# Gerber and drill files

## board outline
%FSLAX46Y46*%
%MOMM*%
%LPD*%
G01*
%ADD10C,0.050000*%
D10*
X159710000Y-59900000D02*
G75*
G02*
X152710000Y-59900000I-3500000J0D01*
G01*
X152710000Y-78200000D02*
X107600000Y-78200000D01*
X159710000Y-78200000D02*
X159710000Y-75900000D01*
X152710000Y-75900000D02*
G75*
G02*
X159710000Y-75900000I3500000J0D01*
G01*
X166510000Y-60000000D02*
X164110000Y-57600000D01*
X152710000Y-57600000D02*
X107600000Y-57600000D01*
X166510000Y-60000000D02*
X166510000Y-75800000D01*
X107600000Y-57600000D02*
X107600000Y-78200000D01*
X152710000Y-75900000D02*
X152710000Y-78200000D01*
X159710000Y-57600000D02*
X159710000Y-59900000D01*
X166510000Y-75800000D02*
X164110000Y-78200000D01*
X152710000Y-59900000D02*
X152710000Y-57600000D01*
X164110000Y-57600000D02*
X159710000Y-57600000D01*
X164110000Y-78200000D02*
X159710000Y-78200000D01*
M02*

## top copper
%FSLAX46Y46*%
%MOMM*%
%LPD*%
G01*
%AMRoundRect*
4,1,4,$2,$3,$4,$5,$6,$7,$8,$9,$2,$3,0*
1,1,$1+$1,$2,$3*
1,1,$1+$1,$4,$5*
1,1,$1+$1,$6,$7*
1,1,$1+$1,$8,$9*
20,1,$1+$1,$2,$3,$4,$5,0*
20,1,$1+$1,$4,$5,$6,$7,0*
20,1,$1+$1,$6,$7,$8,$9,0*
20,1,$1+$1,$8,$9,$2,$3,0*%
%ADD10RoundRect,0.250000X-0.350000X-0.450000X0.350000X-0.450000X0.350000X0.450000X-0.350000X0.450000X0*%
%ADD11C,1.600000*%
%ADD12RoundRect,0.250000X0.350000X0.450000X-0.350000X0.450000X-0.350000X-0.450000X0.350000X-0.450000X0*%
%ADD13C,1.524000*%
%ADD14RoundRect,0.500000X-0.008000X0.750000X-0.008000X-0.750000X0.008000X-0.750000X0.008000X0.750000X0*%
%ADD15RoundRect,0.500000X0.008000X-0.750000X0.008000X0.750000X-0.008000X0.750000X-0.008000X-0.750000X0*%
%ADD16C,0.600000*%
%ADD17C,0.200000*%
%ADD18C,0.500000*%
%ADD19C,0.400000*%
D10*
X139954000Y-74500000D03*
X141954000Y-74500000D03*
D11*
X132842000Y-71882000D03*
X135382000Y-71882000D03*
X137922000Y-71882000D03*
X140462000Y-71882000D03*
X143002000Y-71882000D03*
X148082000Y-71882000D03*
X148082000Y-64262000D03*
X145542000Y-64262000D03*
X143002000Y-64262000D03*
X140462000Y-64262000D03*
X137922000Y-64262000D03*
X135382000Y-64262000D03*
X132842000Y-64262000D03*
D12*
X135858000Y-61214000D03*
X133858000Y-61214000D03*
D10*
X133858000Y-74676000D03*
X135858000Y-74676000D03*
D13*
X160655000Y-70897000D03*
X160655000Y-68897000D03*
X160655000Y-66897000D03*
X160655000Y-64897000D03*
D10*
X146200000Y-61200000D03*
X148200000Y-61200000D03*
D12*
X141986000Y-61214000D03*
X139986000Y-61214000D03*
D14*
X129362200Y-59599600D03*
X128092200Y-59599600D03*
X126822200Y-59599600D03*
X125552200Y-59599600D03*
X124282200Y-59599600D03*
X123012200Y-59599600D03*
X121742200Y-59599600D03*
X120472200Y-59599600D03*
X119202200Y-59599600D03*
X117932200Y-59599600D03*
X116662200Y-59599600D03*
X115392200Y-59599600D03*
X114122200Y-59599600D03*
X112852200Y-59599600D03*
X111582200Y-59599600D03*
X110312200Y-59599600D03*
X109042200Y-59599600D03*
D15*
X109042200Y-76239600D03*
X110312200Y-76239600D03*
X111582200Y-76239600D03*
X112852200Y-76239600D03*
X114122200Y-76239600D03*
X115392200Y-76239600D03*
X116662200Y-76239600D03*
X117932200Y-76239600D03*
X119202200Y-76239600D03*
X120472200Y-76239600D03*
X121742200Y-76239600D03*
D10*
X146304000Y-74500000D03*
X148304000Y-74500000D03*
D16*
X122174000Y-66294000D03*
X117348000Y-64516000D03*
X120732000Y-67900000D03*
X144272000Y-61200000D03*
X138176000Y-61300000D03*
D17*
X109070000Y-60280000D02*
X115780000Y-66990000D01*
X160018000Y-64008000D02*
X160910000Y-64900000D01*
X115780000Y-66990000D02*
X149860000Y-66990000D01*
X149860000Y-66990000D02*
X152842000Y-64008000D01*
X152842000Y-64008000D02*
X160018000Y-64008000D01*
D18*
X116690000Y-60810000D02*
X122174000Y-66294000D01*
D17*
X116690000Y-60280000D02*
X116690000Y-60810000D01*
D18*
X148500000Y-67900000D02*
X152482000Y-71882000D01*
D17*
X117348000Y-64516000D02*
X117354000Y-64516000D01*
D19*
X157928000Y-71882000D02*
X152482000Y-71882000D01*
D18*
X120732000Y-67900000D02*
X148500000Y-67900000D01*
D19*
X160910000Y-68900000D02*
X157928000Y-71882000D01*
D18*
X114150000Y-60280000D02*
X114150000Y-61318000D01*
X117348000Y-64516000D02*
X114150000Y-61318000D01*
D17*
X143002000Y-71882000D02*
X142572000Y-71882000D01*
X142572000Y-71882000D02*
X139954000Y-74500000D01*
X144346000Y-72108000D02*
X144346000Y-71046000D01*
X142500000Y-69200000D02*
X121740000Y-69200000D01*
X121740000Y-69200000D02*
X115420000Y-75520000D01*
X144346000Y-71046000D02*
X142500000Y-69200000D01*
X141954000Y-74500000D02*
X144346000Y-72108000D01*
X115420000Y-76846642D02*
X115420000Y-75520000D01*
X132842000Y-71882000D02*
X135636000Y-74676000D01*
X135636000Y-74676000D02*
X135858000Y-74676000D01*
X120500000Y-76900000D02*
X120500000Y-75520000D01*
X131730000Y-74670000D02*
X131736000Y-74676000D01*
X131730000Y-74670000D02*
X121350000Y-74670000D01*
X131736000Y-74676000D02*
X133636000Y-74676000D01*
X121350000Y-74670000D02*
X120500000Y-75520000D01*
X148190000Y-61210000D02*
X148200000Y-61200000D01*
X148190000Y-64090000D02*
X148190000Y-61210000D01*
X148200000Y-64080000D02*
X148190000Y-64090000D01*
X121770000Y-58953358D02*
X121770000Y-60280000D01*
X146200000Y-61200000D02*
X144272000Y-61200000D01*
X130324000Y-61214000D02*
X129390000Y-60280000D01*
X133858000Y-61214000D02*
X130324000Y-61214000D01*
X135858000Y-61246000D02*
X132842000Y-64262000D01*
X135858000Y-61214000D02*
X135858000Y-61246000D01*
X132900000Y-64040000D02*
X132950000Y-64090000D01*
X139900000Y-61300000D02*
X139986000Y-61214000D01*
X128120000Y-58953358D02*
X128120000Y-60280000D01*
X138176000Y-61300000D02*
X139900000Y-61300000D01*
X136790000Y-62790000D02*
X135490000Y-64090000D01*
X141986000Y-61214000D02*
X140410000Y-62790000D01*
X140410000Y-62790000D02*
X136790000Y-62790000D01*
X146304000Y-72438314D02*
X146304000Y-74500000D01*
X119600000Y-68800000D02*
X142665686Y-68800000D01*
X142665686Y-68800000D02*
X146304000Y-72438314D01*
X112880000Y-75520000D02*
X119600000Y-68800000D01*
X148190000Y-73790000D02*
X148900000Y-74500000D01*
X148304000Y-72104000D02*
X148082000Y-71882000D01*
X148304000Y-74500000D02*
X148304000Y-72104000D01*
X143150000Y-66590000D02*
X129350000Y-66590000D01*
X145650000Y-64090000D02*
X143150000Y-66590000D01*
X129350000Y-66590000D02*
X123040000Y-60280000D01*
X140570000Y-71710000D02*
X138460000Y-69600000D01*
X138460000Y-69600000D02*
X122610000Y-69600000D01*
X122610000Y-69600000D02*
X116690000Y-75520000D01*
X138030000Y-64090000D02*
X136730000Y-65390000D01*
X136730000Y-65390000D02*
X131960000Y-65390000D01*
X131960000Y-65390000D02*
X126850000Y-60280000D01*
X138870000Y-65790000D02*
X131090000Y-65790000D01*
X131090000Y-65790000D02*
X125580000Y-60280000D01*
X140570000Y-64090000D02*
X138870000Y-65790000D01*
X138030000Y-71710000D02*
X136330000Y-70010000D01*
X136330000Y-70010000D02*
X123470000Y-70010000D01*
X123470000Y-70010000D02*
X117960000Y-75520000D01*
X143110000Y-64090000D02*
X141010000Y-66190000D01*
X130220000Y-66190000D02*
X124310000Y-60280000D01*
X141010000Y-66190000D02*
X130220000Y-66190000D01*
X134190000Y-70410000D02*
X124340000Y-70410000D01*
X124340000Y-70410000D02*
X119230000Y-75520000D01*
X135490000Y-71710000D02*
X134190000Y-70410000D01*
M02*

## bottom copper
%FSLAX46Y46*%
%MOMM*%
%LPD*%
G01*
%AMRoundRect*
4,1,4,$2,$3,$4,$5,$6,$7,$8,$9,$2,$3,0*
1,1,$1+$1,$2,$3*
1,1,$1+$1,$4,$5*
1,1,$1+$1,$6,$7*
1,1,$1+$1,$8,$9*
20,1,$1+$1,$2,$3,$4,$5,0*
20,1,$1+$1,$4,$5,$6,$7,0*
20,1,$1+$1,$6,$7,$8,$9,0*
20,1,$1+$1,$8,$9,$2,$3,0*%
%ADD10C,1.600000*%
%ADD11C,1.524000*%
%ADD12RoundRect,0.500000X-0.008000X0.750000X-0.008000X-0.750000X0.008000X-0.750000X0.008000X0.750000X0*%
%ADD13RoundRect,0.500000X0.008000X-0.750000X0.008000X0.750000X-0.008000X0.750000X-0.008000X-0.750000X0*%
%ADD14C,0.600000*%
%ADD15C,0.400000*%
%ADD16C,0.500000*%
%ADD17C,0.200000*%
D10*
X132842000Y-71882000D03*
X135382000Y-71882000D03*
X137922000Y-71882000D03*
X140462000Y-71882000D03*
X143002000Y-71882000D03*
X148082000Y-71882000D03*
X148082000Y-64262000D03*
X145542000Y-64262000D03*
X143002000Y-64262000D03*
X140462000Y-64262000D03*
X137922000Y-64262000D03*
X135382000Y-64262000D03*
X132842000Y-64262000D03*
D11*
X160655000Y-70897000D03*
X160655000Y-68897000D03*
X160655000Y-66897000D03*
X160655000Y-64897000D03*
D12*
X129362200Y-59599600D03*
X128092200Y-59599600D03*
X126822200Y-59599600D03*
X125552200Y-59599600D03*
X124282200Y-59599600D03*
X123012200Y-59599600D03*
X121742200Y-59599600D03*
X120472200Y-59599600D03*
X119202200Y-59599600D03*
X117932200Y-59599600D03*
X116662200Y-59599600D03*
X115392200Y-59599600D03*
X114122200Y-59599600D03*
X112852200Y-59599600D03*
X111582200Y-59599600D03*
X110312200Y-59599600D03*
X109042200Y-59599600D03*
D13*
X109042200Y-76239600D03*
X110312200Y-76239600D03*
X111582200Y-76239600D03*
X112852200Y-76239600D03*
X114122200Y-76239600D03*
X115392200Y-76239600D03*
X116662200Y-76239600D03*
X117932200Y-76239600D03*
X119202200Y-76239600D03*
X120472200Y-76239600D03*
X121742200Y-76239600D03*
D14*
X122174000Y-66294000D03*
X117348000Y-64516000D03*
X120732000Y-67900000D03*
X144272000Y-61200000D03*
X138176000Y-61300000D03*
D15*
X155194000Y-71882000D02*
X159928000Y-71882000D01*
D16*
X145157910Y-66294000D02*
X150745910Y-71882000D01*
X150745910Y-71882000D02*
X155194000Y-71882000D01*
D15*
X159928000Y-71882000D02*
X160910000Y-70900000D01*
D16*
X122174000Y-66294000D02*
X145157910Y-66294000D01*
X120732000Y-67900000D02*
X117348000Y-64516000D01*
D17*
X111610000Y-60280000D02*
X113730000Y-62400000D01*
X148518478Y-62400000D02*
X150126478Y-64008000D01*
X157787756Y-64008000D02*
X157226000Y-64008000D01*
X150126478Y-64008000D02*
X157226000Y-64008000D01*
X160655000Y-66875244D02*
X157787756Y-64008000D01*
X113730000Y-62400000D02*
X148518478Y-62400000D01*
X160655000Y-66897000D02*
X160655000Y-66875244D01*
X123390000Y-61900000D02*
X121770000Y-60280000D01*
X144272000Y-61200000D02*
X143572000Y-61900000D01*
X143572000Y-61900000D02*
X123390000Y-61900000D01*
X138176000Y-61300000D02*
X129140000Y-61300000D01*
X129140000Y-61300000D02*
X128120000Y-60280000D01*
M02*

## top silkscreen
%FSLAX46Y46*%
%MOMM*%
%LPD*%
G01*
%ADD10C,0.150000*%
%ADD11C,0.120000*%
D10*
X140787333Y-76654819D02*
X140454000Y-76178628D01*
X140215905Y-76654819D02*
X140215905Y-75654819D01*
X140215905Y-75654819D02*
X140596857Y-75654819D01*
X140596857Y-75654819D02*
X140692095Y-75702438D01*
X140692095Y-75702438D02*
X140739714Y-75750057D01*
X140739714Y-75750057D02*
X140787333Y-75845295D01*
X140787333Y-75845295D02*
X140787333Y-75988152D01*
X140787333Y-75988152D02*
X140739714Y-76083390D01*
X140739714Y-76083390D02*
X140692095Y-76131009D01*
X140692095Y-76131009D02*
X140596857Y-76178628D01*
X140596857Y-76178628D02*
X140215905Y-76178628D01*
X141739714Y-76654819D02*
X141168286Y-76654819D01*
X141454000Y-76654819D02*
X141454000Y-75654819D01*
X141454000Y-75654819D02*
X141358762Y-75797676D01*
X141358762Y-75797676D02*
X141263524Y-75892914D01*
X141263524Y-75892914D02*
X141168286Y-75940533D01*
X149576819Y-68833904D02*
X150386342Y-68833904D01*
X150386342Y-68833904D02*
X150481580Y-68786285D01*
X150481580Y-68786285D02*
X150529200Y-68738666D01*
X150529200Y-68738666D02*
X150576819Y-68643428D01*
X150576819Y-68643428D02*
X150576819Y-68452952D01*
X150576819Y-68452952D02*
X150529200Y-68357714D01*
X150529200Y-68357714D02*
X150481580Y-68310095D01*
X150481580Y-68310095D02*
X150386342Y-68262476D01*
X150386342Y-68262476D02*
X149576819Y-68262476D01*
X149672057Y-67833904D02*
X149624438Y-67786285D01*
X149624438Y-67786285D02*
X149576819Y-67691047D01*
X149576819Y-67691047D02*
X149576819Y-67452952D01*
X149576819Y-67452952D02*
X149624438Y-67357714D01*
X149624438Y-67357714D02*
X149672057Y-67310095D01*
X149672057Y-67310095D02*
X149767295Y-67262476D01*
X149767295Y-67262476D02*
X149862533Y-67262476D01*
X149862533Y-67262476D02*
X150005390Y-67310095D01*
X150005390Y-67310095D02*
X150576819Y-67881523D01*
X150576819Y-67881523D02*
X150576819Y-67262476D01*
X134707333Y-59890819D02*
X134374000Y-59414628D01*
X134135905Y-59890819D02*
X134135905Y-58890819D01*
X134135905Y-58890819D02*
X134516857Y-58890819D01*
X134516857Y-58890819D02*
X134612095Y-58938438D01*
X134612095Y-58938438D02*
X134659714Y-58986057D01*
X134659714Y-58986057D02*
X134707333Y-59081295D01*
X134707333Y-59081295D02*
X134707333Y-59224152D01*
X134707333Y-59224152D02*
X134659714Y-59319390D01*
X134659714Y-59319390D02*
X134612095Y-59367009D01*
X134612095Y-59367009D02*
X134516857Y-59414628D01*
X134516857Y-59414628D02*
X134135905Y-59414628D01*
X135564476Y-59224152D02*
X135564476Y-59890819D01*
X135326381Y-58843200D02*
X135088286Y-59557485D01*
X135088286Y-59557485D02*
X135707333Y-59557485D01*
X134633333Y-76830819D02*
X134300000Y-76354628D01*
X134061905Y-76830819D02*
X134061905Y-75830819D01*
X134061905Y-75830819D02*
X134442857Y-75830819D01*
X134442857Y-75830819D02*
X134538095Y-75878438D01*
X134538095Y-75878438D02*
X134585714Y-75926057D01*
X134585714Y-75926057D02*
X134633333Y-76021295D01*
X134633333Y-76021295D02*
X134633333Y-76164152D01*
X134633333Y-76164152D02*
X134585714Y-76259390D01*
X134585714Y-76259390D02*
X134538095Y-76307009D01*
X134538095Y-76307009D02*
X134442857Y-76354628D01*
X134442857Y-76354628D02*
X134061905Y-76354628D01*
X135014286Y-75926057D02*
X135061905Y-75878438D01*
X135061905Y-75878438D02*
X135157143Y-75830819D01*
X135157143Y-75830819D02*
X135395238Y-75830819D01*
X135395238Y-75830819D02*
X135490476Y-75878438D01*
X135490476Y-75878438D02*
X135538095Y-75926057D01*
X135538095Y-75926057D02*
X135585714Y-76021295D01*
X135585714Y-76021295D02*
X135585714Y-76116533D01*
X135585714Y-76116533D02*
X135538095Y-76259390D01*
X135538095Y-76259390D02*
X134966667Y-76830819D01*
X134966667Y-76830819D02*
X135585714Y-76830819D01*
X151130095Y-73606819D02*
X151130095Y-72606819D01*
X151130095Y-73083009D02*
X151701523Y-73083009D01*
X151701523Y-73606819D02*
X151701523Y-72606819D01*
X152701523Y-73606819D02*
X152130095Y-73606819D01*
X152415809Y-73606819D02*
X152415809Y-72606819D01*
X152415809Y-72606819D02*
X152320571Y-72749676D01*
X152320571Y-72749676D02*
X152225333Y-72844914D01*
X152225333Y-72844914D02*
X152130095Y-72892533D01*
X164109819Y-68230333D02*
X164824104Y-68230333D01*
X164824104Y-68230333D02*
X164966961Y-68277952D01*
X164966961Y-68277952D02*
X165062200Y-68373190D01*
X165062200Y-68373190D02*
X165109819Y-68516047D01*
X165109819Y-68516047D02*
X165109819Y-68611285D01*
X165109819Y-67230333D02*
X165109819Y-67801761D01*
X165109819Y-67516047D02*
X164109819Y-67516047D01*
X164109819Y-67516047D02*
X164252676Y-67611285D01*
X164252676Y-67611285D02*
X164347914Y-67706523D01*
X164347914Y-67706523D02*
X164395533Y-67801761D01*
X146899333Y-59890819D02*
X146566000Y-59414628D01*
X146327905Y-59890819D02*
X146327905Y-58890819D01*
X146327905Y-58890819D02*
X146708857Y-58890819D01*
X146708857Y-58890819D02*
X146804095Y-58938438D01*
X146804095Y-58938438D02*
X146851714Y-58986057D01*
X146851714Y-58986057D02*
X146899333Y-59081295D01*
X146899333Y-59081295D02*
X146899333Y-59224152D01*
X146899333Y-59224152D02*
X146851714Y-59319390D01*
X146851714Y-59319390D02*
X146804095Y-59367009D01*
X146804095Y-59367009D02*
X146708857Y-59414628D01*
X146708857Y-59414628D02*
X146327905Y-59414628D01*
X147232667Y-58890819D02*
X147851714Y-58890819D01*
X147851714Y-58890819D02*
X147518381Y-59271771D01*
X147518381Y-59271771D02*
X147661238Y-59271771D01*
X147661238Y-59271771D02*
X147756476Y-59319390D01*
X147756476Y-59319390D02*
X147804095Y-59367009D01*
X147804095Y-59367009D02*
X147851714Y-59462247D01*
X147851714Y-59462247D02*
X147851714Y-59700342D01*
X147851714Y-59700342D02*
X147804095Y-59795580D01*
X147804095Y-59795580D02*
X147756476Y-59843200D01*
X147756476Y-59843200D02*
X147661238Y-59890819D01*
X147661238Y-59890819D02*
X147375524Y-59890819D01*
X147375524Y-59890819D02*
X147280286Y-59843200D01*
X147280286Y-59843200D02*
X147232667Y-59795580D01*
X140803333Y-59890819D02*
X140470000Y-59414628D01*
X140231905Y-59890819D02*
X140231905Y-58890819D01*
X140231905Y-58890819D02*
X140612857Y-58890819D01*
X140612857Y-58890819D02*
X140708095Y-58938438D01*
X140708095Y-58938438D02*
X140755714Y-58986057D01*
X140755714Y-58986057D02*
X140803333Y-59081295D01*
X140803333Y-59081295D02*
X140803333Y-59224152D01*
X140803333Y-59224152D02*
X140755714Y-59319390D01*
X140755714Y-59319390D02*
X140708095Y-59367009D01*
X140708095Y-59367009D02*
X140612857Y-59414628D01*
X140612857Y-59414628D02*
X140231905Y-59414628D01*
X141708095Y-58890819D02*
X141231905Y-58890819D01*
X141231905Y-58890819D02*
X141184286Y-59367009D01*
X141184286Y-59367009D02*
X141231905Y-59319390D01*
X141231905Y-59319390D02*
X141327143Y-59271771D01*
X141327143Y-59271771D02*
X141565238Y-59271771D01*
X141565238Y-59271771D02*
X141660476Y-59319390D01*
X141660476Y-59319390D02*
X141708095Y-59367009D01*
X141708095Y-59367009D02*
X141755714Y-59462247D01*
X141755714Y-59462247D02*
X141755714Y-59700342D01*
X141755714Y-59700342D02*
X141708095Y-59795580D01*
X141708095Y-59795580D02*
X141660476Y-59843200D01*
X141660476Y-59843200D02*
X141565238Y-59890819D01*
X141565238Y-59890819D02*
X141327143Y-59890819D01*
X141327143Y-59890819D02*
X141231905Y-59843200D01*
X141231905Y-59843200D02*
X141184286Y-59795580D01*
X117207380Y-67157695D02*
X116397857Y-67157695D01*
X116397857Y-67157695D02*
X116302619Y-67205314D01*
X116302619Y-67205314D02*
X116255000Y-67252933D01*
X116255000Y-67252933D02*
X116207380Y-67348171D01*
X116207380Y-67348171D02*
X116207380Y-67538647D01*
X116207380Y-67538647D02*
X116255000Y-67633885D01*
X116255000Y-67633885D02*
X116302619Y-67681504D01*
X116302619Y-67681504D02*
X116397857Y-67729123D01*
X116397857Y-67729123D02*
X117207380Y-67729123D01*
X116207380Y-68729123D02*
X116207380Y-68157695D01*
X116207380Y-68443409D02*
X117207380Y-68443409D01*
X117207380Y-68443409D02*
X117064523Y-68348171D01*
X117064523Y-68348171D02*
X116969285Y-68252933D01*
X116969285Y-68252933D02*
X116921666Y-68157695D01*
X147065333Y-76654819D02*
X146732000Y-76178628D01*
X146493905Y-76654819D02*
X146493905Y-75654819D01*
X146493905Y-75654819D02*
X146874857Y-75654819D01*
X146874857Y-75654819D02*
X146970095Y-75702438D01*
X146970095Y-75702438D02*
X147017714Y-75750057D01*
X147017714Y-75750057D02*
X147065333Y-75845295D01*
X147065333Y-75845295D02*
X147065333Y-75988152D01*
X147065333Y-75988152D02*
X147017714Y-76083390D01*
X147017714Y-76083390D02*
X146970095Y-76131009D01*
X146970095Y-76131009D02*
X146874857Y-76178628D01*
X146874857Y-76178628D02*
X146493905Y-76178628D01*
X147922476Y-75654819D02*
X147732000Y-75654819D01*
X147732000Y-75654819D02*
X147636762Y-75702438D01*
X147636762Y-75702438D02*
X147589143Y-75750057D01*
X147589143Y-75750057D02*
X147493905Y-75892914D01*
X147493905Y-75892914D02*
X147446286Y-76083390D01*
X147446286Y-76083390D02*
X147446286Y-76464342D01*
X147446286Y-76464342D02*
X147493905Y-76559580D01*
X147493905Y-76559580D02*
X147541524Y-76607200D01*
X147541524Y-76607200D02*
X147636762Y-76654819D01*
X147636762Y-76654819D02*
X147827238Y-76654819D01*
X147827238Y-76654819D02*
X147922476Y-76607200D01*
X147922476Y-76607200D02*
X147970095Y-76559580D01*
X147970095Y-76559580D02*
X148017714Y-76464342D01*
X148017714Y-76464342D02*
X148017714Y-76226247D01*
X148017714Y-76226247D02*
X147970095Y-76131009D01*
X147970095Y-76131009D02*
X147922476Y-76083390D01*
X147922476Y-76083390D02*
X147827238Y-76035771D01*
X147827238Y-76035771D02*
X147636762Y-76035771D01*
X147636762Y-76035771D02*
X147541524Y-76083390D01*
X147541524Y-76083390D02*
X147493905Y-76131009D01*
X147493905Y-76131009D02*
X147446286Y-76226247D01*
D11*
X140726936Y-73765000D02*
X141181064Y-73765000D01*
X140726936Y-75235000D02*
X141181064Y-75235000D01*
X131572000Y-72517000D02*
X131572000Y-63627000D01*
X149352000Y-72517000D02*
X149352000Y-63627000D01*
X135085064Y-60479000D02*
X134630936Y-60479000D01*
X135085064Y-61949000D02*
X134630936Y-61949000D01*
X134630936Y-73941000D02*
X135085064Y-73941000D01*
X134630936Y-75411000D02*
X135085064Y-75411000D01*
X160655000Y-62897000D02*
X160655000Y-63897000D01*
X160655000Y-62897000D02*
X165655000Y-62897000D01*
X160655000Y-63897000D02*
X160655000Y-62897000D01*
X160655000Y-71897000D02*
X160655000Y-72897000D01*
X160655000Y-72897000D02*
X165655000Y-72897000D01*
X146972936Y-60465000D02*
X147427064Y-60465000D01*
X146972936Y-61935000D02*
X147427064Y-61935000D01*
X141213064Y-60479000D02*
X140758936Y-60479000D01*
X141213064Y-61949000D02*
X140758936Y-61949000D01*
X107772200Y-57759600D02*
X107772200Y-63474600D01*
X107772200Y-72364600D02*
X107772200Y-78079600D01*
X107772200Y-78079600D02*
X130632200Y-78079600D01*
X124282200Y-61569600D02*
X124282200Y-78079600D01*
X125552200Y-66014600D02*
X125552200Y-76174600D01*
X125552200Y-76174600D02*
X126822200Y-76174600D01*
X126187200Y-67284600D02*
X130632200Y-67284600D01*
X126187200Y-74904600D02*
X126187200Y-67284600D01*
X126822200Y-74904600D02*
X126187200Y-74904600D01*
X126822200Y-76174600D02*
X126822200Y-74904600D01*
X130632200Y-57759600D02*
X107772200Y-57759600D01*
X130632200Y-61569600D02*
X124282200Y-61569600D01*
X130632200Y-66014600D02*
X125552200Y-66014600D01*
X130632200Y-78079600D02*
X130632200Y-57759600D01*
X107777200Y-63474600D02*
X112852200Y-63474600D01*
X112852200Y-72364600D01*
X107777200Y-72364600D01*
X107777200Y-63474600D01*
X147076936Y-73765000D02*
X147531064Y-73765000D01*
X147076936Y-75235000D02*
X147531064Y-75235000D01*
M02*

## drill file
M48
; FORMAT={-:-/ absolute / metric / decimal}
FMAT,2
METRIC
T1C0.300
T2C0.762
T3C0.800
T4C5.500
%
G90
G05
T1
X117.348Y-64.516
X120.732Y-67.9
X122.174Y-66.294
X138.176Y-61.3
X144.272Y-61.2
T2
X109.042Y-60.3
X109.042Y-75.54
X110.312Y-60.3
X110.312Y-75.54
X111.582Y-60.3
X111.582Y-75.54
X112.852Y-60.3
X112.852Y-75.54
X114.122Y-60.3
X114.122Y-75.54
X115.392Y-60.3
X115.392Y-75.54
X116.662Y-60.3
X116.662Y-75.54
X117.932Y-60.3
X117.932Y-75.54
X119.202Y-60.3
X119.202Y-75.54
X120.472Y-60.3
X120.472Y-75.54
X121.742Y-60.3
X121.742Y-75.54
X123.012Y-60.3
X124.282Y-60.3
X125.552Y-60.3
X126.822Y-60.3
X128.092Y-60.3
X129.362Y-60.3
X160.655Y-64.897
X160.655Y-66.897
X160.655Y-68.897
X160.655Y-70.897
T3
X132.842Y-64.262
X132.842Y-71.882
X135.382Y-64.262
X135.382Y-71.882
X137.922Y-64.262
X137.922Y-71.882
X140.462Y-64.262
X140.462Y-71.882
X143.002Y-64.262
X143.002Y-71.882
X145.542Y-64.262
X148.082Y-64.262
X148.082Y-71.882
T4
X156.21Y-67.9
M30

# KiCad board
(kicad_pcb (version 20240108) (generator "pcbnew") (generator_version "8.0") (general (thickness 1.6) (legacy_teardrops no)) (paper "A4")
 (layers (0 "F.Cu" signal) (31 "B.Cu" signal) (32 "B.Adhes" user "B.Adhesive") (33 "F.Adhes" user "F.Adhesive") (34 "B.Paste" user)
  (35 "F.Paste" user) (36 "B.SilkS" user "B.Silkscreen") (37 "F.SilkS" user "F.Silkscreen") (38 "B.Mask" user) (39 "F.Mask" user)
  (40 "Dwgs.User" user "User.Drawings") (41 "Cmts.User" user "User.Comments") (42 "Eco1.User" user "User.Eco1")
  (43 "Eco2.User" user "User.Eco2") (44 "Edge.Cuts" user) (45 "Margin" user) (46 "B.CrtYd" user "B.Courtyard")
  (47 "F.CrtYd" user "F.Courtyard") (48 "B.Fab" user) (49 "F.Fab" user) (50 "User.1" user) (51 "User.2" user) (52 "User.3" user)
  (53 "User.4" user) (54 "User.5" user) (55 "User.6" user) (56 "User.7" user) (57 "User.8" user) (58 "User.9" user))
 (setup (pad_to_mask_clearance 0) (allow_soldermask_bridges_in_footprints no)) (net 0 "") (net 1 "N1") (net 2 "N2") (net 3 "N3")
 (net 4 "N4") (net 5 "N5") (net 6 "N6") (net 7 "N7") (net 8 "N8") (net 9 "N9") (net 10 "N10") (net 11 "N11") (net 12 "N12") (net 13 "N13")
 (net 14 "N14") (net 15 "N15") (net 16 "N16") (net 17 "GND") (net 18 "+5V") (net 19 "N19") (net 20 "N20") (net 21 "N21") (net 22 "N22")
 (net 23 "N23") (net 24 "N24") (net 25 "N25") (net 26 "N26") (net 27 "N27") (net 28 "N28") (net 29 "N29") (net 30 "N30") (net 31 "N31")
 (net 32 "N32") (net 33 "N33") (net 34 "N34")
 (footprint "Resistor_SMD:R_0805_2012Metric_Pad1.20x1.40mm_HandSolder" (layer "F.Cu") (at 140.954 74.5)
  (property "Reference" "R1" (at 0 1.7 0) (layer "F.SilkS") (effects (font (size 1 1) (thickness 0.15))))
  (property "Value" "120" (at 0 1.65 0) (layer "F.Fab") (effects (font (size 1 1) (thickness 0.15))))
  (fp_line (start -0.227064 -0.735) (end 0.227064 -0.735) (stroke (width 0.12) (type solid)) (layer "F.SilkS"))
  (fp_line (start -0.227064 0.735) (end 0.227064 0.735) (stroke (width 0.12) (type solid)) (layer "F.SilkS"))
  (pad "1" smd roundrect (at -1 0) (size 1.2 1.4) (layers "F.Cu" "F.Paste" "F.Mask") (roundrect_rratio 0.208333) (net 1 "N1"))
  (pad "2" smd roundrect (at 1 0) (size 1.2 1.4) (layers "F.Cu" "F.Paste" "F.Mask") (roundrect_rratio 0.208333) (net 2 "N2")))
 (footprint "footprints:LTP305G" (layer "F.Cu") (at 150.622 68.072 90)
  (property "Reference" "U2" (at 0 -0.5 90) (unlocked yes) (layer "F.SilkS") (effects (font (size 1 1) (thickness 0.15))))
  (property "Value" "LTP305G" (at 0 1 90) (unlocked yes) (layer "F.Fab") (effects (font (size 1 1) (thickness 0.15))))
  (fp_line (start -4.445 -19.05) (end 4.445 -19.05) (stroke (width 0.12) (type default)) (layer "F.SilkS"))
  (fp_line (start -4.445 -1.27) (end 4.445 -1.27) (stroke (width 0.12) (type default)) (layer "F.SilkS"))
  (pad "1" thru_hole circle (at -3.81 -17.78 90) (size 1.6 1.6) (drill 0.8) (layers "*.Cu" "*.Mask") (remove_unused_layers no) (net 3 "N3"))
  (pad "2" thru_hole circle (at -3.81 -15.24 90) (size 1.6 1.6) (drill 0.8) (layers "*.Cu" "*.Mask") (remove_unused_layers no) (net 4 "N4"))
  (pad "3" thru_hole circle (at -3.81 -12.7 90) (size 1.6 1.6) (drill 0.8) (layers "*.Cu" "*.Mask") (remove_unused_layers no) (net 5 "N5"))
  (pad "4" thru_hole circle (at -3.81 -10.16 90) (size 1.6 1.6) (drill 0.8) (layers "*.Cu" "*.Mask") (remove_unused_layers no) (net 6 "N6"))
  (pad "5" thru_hole circle (at -3.81 -7.62 90) (size 1.6 1.6) (drill 0.8) (layers "*.Cu" "*.Mask") (remove_unused_layers no) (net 1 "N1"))
  (pad "7" thru_hole circle (at -3.81 -2.54 90) (size 1.6 1.6) (drill 0.8) (layers "*.Cu" "*.Mask") (remove_unused_layers no) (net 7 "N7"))
  (pad "8" thru_hole circle (at 3.81 -2.54 90) (size 1.6 1.6) (drill 0.8) (layers "*.Cu" "*.Mask") (remove_unused_layers no) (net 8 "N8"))
  (pad "9" thru_hole circle (at 3.81 -5.08 90) (size 1.6 1.6) (drill 0.8) (layers "*.Cu" "*.Mask") (remove_unused_layers no) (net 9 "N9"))
  (pad "10" thru_hole circle (at 3.81 -7.62 90) (size 1.6 1.6) (drill 0.8) (layers "*.Cu" "*.Mask") (remove_unused_layers no) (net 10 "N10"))
  (pad "11" thru_hole circle (at 3.81 -10.16 90) (size 1.6 1.6) (drill 0.8) (layers "*.Cu" "*.Mask") (remove_unused_layers no)
   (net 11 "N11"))
  (pad "12" thru_hole circle (at 3.81 -12.7 90) (size 1.6 1.6) (drill 0.8) (layers "*.Cu" "*.Mask") (remove_unused_layers no) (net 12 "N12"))
  (pad "13" thru_hole circle (at 3.81 -15.24 90) (size 1.6 1.6) (drill 0.8) (layers "*.Cu" "*.Mask") (remove_unused_layers no)
   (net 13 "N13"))
  (pad "14" thru_hole circle (at 3.81 -17.78 90) (size 1.6 1.6) (drill 0.8) (layers "*.Cu" "*.Mask") (remove_unused_layers no)
   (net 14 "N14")))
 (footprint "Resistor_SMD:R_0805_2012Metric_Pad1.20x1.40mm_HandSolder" (layer "F.Cu") (at 134.858 61.214 180)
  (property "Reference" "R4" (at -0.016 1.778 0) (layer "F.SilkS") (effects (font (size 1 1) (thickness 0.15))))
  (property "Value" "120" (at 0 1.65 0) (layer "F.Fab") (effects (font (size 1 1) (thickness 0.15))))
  (fp_line (start -0.227064 0.735) (end 0.227064 0.735) (stroke (width 0.12) (type solid)) (layer "F.SilkS"))
  (fp_line (start -0.227064 -0.735) (end 0.227064 -0.735) (stroke (width 0.12) (type solid)) (layer "F.SilkS"))
  (pad "1" smd roundrect (at -1 0 180) (size 1.2 1.4) (layers "F.Cu" "F.Paste" "F.Mask") (roundrect_rratio 0.208333) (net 14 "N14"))
  (pad "2" smd roundrect (at 1 0 180) (size 1.2 1.4) (layers "F.Cu" "F.Paste" "F.Mask") (roundrect_rratio 0.208333) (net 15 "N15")))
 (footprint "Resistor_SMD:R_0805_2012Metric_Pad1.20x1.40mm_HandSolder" (layer "F.Cu") (at 134.858 74.676)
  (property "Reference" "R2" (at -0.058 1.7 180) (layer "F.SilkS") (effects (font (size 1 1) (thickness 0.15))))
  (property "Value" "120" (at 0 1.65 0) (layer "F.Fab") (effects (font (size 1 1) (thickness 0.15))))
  (fp_line (start -0.227064 -0.735) (end 0.227064 -0.735) (stroke (width 0.12) (type solid)) (layer "F.SilkS"))
  (fp_line (start -0.227064 0.735) (end 0.227064 0.735) (stroke (width 0.12) (type solid)) (layer "F.SilkS"))
  (pad "1" smd roundrect (at -1 0) (size 1.2 1.4) (layers "F.Cu" "F.Paste" "F.Mask") (roundrect_rratio 0.208333) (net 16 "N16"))
  (pad "2" smd roundrect (at 1 0) (size 1.2 1.4) (layers "F.Cu" "F.Paste" "F.Mask") (roundrect_rratio 0.208333) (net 3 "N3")))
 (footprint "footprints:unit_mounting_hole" (layer "F.Cu") (at 156.21 75.4)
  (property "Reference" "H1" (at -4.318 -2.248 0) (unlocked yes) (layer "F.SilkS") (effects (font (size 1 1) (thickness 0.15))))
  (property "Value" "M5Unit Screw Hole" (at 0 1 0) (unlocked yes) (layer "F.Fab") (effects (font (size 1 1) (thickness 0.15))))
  (pad "" np_thru_hole circle (at 0 -7.5) (size 5.5 5.5) (drill 5.5) (layers "F&B.Cu" "*.Mask")))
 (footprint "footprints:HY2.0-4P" (layer "F.Cu") (at 165.655 67.897 90)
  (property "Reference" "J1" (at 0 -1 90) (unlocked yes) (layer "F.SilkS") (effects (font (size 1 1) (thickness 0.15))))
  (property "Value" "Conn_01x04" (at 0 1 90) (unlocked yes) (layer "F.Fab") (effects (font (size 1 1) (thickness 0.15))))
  (fp_line (start 5 -5) (end 4 -5) (stroke (width 0.12) (type default)) (layer "F.SilkS"))
  (fp_line (start 5 -5) (end 5 0) (stroke (width 0.12) (type default)) (layer "F.SilkS"))
  (fp_line (start 4 -5) (end 5 -5) (stroke (width 0.12) (type default)) (layer "F.SilkS"))
  (fp_line (start -4 -5) (end -5 -5) (stroke (width 0.12) (type default)) (layer "F.SilkS"))
  (fp_line (start -5 -5) (end -5 0) (stroke (width 0.12) (type default)) (layer "F.SilkS"))
  (pad "1" thru_hole circle (at -3 -5 90) (size 1.524 1.524) (drill 0.762) (layers "*.Cu" "*.Mask") (remove_unused_layers no) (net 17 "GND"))
  (pad "2" thru_hole circle (at -1 -5 90) (size 1.524 1.524) (drill 0.762) (layers "*.Cu" "*.Mask") (remove_unused_layers no) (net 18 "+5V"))
  (pad "3" thru_hole circle (at 1 -5 90) (size 1.524 1.524) (drill 0.762) (layers "*.Cu" "*.Mask") (remove_unused_layers no) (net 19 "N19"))
  (pad "4" thru_hole circle (at 3 -5 90) (size 1.524 1.524) (drill 0.762) (layers "*.Cu" "*.Mask") (remove_unused_layers no) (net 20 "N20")))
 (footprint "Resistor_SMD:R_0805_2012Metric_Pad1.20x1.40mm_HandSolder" (layer "F.Cu") (at 147.2 61.2)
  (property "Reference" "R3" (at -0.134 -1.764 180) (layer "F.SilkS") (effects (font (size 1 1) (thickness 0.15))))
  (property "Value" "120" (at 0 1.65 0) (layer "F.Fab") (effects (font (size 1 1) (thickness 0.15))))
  (fp_line (start -0.227064 -0.735) (end 0.227064 -0.735) (stroke (width 0.12) (type solid)) (layer "F.SilkS"))
  (fp_line (start -0.227064 0.735) (end 0.227064 0.735) (stroke (width 0.12) (type solid)) (layer "F.SilkS"))
  (pad "1" smd roundrect (at -1 0) (size 1.2 1.4) (layers "F.Cu" "F.Paste" "F.Mask") (roundrect_rratio 0.208333) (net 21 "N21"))
  (pad "2" smd roundrect (at 1 0) (size 1.2 1.4) (layers "F.Cu" "F.Paste" "F.Mask") (roundrect_rratio 0.208333) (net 8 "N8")))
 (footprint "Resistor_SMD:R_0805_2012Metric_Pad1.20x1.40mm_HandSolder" (layer "F.Cu") (at 140.986 61.214 180)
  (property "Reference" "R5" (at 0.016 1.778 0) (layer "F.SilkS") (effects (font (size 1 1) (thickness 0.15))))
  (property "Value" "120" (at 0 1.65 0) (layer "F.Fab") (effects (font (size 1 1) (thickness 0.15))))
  (fp_line (start -0.227064 0.735) (end 0.227064 0.735) (stroke (width 0.12) (type solid)) (layer "F.SilkS"))
  (fp_line (start -0.227064 -0.735) (end 0.227064 -0.735) (stroke (width 0.12) (type solid)) (layer "F.SilkS"))
  (pad "1" smd roundrect (at -1 0 180) (size 1.2 1.4) (layers "F.Cu" "F.Paste" "F.Mask") (roundrect_rratio 0.208333) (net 13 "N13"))
  (pad "2" smd roundrect (at 1 0 180) (size 1.2 1.4) (layers "F.Cu" "F.Paste" "F.Mask") (roundrect_rratio 0.208333) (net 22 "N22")))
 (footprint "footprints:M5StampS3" (layer "F.Cu") (at 106.5022 67.9196 -90)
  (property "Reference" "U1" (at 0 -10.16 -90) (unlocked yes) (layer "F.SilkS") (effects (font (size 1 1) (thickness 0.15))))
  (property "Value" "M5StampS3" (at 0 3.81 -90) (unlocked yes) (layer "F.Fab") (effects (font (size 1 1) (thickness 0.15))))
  (fp_line (start -10.16 -1.27) (end -4.445 -1.27) (stroke (width 0.12) (type default)) (layer "F.SilkS"))
  (fp_line (start 4.445 -1.27) (end 10.16 -1.27) (stroke (width 0.12) (type default)) (layer "F.SilkS"))
  (fp_line (start 10.16 -1.27) (end 10.16 -24.13) (stroke (width 0.12) (type default)) (layer "F.SilkS"))
  (fp_line (start -6.35 -17.78) (end 10.16 -17.78) (stroke (width 0.12) (type default)) (layer "F.SilkS"))
  (fp_line (start -1.905 -19.05) (end 8.255 -19.05) (stroke (width 0.12) (type default)) (layer "F.SilkS"))
  (fp_line (start 8.255 -19.05) (end 8.255 -20.32) (stroke (width 0.12) (type default)) (layer "F.SilkS"))
  (fp_line (start -0.635 -19.685) (end -0.635 -24.13) (stroke (width 0.12) (type default)) (layer "F.SilkS"))
  (fp_line (start 6.985 -19.685) (end -0.635 -19.685) (stroke (width 0.12) (type default)) (layer "F.SilkS"))
  (fp_line (start 6.985 -20.32) (end 6.985 -19.685) (stroke (width 0.12) (type default)) (layer "F.SilkS"))
  (fp_line (start 8.255 -20.32) (end 6.985 -20.32) (stroke (width 0.12) (type default)) (layer "F.SilkS"))
  (fp_line (start -10.16 -24.13) (end -10.16 -1.27) (stroke (width 0.12) (type default)) (layer "F.SilkS"))
  (fp_line (start -6.35 -24.13) (end -6.35 -17.78) (stroke (width 0.12) (type default)) (layer "F.SilkS"))
  (fp_line (start -1.905 -24.13) (end -1.905 -19.05) (stroke (width 0.12) (type default)) (layer "F.SilkS"))
  (fp_line (start 10.16 -24.13) (end -10.16 -24.13) (stroke (width 0.12) (type default)) (layer "F.SilkS"))
  (fp_rect (start -4.445 -6.35) (end 4.445 -1.275) (stroke (width 0.12) (type default)) (fill none) (layer "F.SilkS"))
  (pad "1" thru_hole roundrect (at -7.62 -22.86 270) (size 2.5 1.016) (drill 0.762 (offset -0.7 0)) (layers "*.Cu" "*.Mask")
   (remove_unused_layers no) (roundrect_rratio 0.4921259843) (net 15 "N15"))
  (pad "2" thru_hole roundrect (at -7.62 -21.59 270) (size 2.5 1.016) (drill 0.762 (offset -0.7 0)) (layers "*.Cu" "*.Mask")
   (remove_unused_layers no) (roundrect_rratio 0.4921259843) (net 22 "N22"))
  (pad "3" thru_hole roundrect (at -7.62 -20.32 270) (size 2.5 1.016) (drill 0.762 (offset -0.7 0)) (layers "*.Cu" "*.Mask")
   (remove_unused_layers no) (roundrect_rratio 0.4921259843) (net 12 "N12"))
  (pad "4" thru_hole roundrect (at -7.62 -19.05 270) (size 2.5 1.016) (drill 0.762 (offset -0.7 0)) (layers "*.Cu" "*.Mask")
   (remove_unused_layers no) (roundrect_rratio 0.4921259843) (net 11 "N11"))
  (pad "5" thru_hole roundrect (at -7.62 -17.78 270) (size 2.5 1.016) (drill 0.762 (offset -0.7 0)) (layers "*.Cu" "*.Mask")
   (remove_unused_layers no) (roundrect_rratio 0.4921259843) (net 10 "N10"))
  (pad "6" thru_hole roundrect (at -7.62 -16.51 270) (size 2.5 1.016) (drill 0.762 (offset -0.7 0)) (layers "*.Cu" "*.Mask")
   (remove_unused_layers no) (roundrect_rratio 0.4921259843) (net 9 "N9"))
  (pad "7" thru_hole roundrect (at -7.62 -15.24 270) (size 2.5 1.016) (drill 0.762 (offset -0.7 0)) (layers "*.Cu" "*.Mask")
   (remove_unused_layers no) (roundrect_rratio 0.4921259843) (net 21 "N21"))
  (pad "8" thru_hole roundrect (at -7.62 -13.97 270) (size 2.5 1.016) (drill 0.762 (offset -0.7 0)) (layers "*.Cu" "*.Mask")
   (remove_unused_layers no) (roundrect_rratio 0.4921259843) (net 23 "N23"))
  (pad "9" thru_hole roundrect (at -7.62 -12.7 270) (size 2.5 1.016) (drill 0.762 (offset -0.7 0)) (layers "*.Cu" "*.Mask")
   (remove_unused_layers no) (roundrect_rratio 0.4921259843) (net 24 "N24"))
  (pad "10" thru_hole roundrect (at -7.62 -11.43 270) (size 2.5 1.016) (drill 0.762 (offset -0.7 0)) (layers "*.Cu" "*.Mask")
   (remove_unused_layers no) (roundrect_rratio 0.4921259843) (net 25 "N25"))
  (pad "11" thru_hole roundrect (at -7.62 -10.16 270) (size 2.5 1.016) (drill 0.762 (offset -0.7 0)) (layers "*.Cu" "*.Mask")
   (remove_unused_layers no) (roundrect_rratio 0.4921259843) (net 17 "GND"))
  (pad "12" thru_hole roundrect (at -7.62 -8.89 270) (size 2.5 1.016) (drill 0.762 (offset -0.7 0)) (layers "*.Cu" "*.Mask")
   (remove_unused_layers no) (roundrect_rratio 0.4921259843) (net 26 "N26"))
  (pad "13" thru_hole roundrect (at -7.62 -7.62 270) (size 2.5 1.016) (drill 0.762 (offset -0.7 0)) (layers "*.Cu" "*.Mask")
   (remove_unused_layers no) (roundrect_rratio 0.4921259843) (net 18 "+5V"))
  (pad "14" thru_hole roundrect (at -7.62 -6.35 270) (size 2.5 1.016) (drill 0.762 (offset -0.7 0)) (layers "*.Cu" "*.Mask")
   (remove_unused_layers no) (roundrect_rratio 0.4921259843) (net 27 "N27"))
  (pad "15" thru_hole roundrect (at -7.62 -5.08 270) (size 2.5 1.016) (drill 0.762 (offset -0.7 0)) (layers "*.Cu" "*.Mask")
   (remove_unused_layers no) (roundrect_rratio 0.4921259843) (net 19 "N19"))
  (pad "16" thru_hole roundrect (at -7.62 -3.81 270) (size 2.5 1.016) (drill 0.762 (offset -0.7 0)) (layers "*.Cu" "*.Mask")
   (remove_unused_layers no) (roundrect_rratio 0.4921259843) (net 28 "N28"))
  (pad "17" thru_hole roundrect (at -7.62 -2.54 270) (size 2.5 1.016) (drill 0.762 (offset -0.7 0)) (layers "*.Cu" "*.Mask")
   (remove_unused_layers no) (roundrect_rratio 0.4921259843) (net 20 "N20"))
  (pad "18" thru_hole roundrect (at 7.62 -2.54 90) (size 2.5 1.016) (drill 0.762 (offset -0.7 0)) (layers "*.Cu" "*.Mask")
   (remove_unused_layers no) (roundrect_rratio 0.4921259843) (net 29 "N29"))
  (pad "19" thru_hole roundrect (at 7.62 -3.81 90) (size 2.5 1.016) (drill 0.762 (offset -0.7 0)) (layers "*.Cu" "*.Mask")
   (remove_unused_layers no) (roundrect_rratio 0.4921259843) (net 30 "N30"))
  (pad "20" thru_hole roundrect (at 7.62 -5.08 90) (size 2.5 1.016) (drill 0.762 (offset -0.7 0)) (layers "*.Cu" "*.Mask")
   (remove_unused_layers no) (roundrect_rratio 0.4921259843) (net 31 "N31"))
  (pad "21" thru_hole roundrect (at 7.62 -6.35 90) (size 2.5 1.016) (drill 0.762 (offset -0.7 0)) (layers "*.Cu" "*.Mask")
   (remove_unused_layers no) (roundrect_rratio 0.4921259843) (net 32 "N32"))
  (pad "22" thru_hole roundrect (at 7.62 -7.62 90) (size 2.5 1.016) (drill 0.762 (offset -0.7 0)) (layers "*.Cu" "*.Mask")
   (remove_unused_layers no) (roundrect_rratio 0.4921259843) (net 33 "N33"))
  (pad "23" thru_hole roundrect (at 7.62 -8.89 90) (size 2.5 1.016) (drill 0.762 (offset -0.7 0)) (layers "*.Cu" "*.Mask")
   (remove_unused_layers no) (roundrect_rratio 0.4921259843) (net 2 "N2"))
  (pad "24" thru_hole roundrect (at 7.62 -10.16 90) (size 2.5 1.016) (drill 0.762 (offset -0.7 0)) (layers "*.Cu" "*.Mask")
   (remove_unused_layers no) (roundrect_rratio 0.4921259843) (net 6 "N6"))
  (pad "25" thru_hole roundrect (at 7.62 -11.43 90) (size 2.5 1.016) (drill 0.762 (offset -0.7 0)) (layers "*.Cu" "*.Mask")
   (remove_unused_layers no) (roundrect_rratio 0.4921259843) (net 5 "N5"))
  (pad "26" thru_hole roundrect (at 7.62 -12.7 90) (size 2.5 1.016) (drill 0.762 (offset -0.7 0)) (layers "*.Cu" "*.Mask")
   (remove_unused_layers no) (roundrect_rratio 0.4921259843) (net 4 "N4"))
  (pad "27" thru_hole roundrect (at 7.62 -13.97 90) (size 2.5 1.016) (drill 0.762 (offset -0.7 0)) (layers "*.Cu" "*.Mask")
   (remove_unused_layers no) (roundrect_rratio 0.4921259843) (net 16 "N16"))
  (pad "28" thru_hole roundrect (at 7.62 -15.24 90) (size 2.5 1.016) (drill 0.762 (offset -0.7 0)) (layers "*.Cu" "*.Mask")
   (remove_unused_layers no) (roundrect_rratio 0.4921259843) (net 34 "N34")))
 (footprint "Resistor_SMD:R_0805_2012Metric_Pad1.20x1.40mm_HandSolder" (layer "F.Cu") (at 147.304 74.5)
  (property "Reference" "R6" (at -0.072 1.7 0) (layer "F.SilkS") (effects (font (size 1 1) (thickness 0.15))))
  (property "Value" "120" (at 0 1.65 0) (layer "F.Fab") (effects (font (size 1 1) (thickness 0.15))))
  (fp_line (start -0.227064 -0.735) (end 0.227064 -0.735) (stroke (width 0.12) (type solid)) (layer "F.SilkS"))
  (fp_line (start -0.227064 0.735) (end 0.227064 0.735) (stroke (width 0.12) (type solid)) (layer "F.SilkS"))
  (pad "1" smd roundrect (at -1 0) (size 1.2 1.4) (layers "F.Cu" "F.Paste" "F.Mask") (roundrect_rratio 0.208333) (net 32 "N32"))
  (pad "2" smd roundrect (at 1 0) (size 1.2 1.4) (layers "F.Cu" "F.Paste" "F.Mask") (roundrect_rratio 0.208333) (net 7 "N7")))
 (gr_arc (start 159.71 59.9) (mid 156.21 63.4) (end 152.71 59.9) (stroke (width 0.05) (type default)) (layer "Edge.Cuts"))
 (gr_line (start 152.71 78.2) (end 107.6 78.2) (stroke (width 0.05) (type default)) (layer "Edge.Cuts"))
 (gr_line (start 159.71 78.2) (end 159.71 75.9) (stroke (width 0.05) (type default)) (layer "Edge.Cuts"))
 (gr_arc (start 152.71 75.9) (mid 156.21 72.4) (end 159.71 75.9) (stroke (width 0.05) (type default)) (layer "Edge.Cuts"))
 (gr_line (start 166.51 60) (end 164.11 57.6) (stroke (width 0.05) (type default)) (layer "Edge.Cuts"))
 (gr_line (start 152.71 57.6) (end 107.6 57.6) (stroke (width 0.05) (type default)) (layer "Edge.Cuts"))
 (gr_line (start 166.51 60) (end 166.51 75.8) (stroke (width 0.05) (type default)) (layer "Edge.Cuts"))
 (gr_line (start 107.6 57.6) (end 107.6 78.2) (stroke (width 0.05) (type default)) (layer "Edge.Cuts"))
 (gr_line (start 152.71 75.9) (end 152.71 78.2) (stroke (width 0.05) (type default)) (layer "Edge.Cuts"))
 (gr_line (start 159.71 57.6) (end 159.71 59.9) (stroke (width 0.05) (type default)) (layer "Edge.Cuts"))
 (gr_line (start 166.51 75.8) (end 164.11 78.2) (stroke (width 0.05) (type default)) (layer "Edge.Cuts"))
 (gr_line (start 152.71 59.9) (end 152.71 57.6) (stroke (width 0.05) (type default)) (layer "Edge.Cuts"))
 (gr_line (start 164.11 57.6) (end 159.71 57.6) (stroke (width 0.05) (type default)) (layer "Edge.Cuts"))
 (gr_line (start 164.11 78.2) (end 159.71 78.2) (stroke (width 0.05) (type default)) (layer "Edge.Cuts"))
 (segment (start 109.07 60.28) (end 115.78 66.99) (width 0.2) (layer "F.Cu") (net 20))
 (segment (start 160.018 64.008) (end 160.91 64.9) (width 0.2) (layer "F.Cu") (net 20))
 (segment (start 115.78 66.99) (end 149.86 66.99) (width 0.2) (layer "F.Cu") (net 20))
 (segment (start 149.86 66.99) (end 152.842 64.008) (width 0.2) (layer "F.Cu") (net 20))
 (segment (start 152.842 64.008) (end 160.018 64.008) (width 0.2) (layer "F.Cu") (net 20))
 (segment (start 116.69 60.81) (end 122.174 66.294) (width 0.5) (layer "F.Cu") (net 17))
 (segment (start 116.69 60.28) (end 116.69 60.81) (width 0.2) (layer "F.Cu") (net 17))
 (via (at 122.174 66.294) (size 0.6) (drill 0.3) (layers "F.Cu" "B.Cu") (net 17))
 (segment (start 155.194 71.882) (end 159.928 71.882) (width 0.4) (layer "B.Cu") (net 17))
 (segment (start 145.15791 66.294) (end 150.74591 71.882) (width 0.5) (layer "B.Cu") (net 17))
 (segment (start 150.74591 71.882) (end 155.194 71.882) (width 0.5) (layer "B.Cu") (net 17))
 (segment (start 159.928 71.882) (end 160.91 70.9) (width 0.4) (layer "B.Cu") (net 17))
 (segment (start 122.174 66.294) (end 145.15791 66.294) (width 0.5) (layer "B.Cu") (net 17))
 (segment (start 148.5 67.9) (end 152.482 71.882) (width 0.5) (layer "F.Cu") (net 18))
 (segment (start 117.348 64.516) (end 117.354 64.516) (width 0.2) (layer "F.Cu") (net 18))
 (segment (start 157.928 71.882) (end 152.482 71.882) (width 0.4) (layer "F.Cu") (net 18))
 (segment (start 120.732 67.9) (end 148.5 67.9) (width 0.5) (layer "F.Cu") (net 18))
 (segment (start 160.91 68.9) (end 157.928 71.882) (width 0.4) (layer "F.Cu") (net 18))
 (segment (start 114.15 60.28) (end 114.15 61.318) (width 0.5) (layer "F.Cu") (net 18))
 (segment (start 117.348 64.516) (end 114.15 61.318) (width 0.5) (layer "F.Cu") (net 18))
 (via (at 117.348 64.516) (size 0.6) (drill 0.3) (layers "F.Cu" "B.Cu") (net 18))
 (via (at 120.732 67.9) (size 0.6) (drill 0.3) (layers "F.Cu" "B.Cu") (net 18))
 (segment (start 120.732 67.9) (end 117.348 64.516) (width 0.5) (layer "B.Cu") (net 18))
 (segment (start 111.61 60.28) (end 113.73 62.4) (width 0.2) (layer "B.Cu") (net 19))
 (segment (start 148.518478 62.4) (end 150.126478 64.008) (width 0.2) (layer "B.Cu") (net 19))
 (segment (start 157.787756 64.008) (end 157.226 64.008) (width 0.2) (layer "B.Cu") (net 19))
 (segment (start 150.126478 64.008) (end 157.226 64.008) (width 0.2) (layer "B.Cu") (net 19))
 (segment (start 160.655 66.875244) (end 157.787756 64.008) (width 0.2) (layer "B.Cu") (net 19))
 (segment (start 113.73 62.4) (end 148.518478 62.4) (width 0.2) (layer "B.Cu") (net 19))
 (segment (start 160.655 66.897) (end 160.655 66.875244) (width 0.2) (layer "B.Cu") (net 19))
 (segment (start 143.002 71.882) (end 142.572 71.882) (width 0.2) (layer "F.Cu") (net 1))
 (segment (start 142.572 71.882) (end 139.954 74.5) (width 0.2) (layer "F.Cu") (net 1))
 (segment (start 144.346 72.108) (end 144.346 71.046) (width 0.2) (layer "F.Cu") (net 2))
 (segment (start 142.5 69.2) (end 121.74 69.2) (width 0.2) (layer "F.Cu") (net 2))
 (segment (start 121.74 69.2) (end 115.42 75.52) (width 0.2) (layer "F.Cu") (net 2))
 (segment (start 144.346 71.046) (end 142.5 69.2) (width 0.2) (layer "F.Cu") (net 2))
 (segment (start 141.954 74.5) (end 144.346 72.108) (width 0.2) (layer "F.Cu") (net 2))
 (segment (start 115.42 76.846642) (end 115.42 75.52) (width 0.2) (layer "F.Cu") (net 2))
 (segment (start 132.842 71.882) (end 135.636 74.676) (width 0.2) (layer "F.Cu") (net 3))
 (segment (start 135.636 74.676) (end 135.858 74.676) (width 0.2) (layer "F.Cu") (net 3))
 (segment (start 120.5 76.9) (end 120.5 75.52) (width 0.2) (layer "F.Cu") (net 16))
 (segment (start 131.73 74.67) (end 131.736 74.676) (width 0.2) (layer "F.Cu") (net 16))
 (segment (start 131.73 74.67) (end 121.35 74.67) (width 0.2) (layer "F.Cu") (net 16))
 (segment (start 131.736 74.676) (end 133.636 74.676) (width 0.2) (layer "F.Cu") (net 16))
 (segment (start 121.35 74.67) (end 120.5 75.52) (width 0.2) (layer "F.Cu") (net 16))
 (segment (start 148.19 61.21) (end 148.2 61.2) (width 0.2) (layer "F.Cu") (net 8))
 (segment (start 148.19 64.09) (end 148.19 61.21) (width 0.2) (layer "F.Cu") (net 8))
 (segment (start 148.2 64.08) (end 148.19 64.09) (width 0.2) (layer "F.Cu") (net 8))
 (segment (start 121.77 58.953358) (end 121.77 60.28) (width 0.2) (layer "F.Cu") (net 21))
 (segment (start 146.2 61.2) (end 144.272 61.2) (width 0.2) (layer "F.Cu") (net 21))
 (via (at 144.272 61.2) (size 0.6) (drill 0.3) (layers "F.Cu" "B.Cu") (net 21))
 (segment (start 123.39 61.9) (end 121.77 60.28) (width 0.2) (layer "B.Cu") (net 21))
 (segment (start 144.272 61.2) (end 143.572 61.9) (width 0.2) (layer "B.Cu") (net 21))
 (segment (start 143.572 61.9) (end 123.39 61.9) (width 0.2) (layer "B.Cu") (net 21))
 (segment (start 130.324 61.214) (end 129.39 60.28) (width 0.2) (layer "F.Cu") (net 15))
 (segment (start 133.858 61.214) (end 130.324 61.214) (width 0.2) (layer "F.Cu") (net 15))
 (segment (start 135.858 61.246) (end 132.842 64.262) (width 0.2) (layer "F.Cu") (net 14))
 (segment (start 135.858 61.214) (end 135.858 61.246) (width 0.2) (layer "F.Cu") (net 14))
 (segment (start 132.9 64.04) (end 132.95 64.09) (width 0.2) (layer "F.Cu") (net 14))
 (segment (start 139.9 61.3) (end 139.986 61.214) (width 0.2) (layer "F.Cu") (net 22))
 (segment (start 128.12 58.953358) (end 128.12 60.28) (width 0.2) (layer "F.Cu") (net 22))
 (segment (start 138.176 61.3) (end 139.9 61.3) (width 0.2) (layer "F.Cu") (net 22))
 (via (at 138.176 61.3) (size 0.6) (drill 0.3) (layers "F.Cu" "B.Cu") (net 22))
 (segment (start 138.176 61.3) (end 129.14 61.3) (width 0.2) (layer "B.Cu") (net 22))
 (segment (start 129.14 61.3) (end 128.12 60.28) (width 0.2) (layer "B.Cu") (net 22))
 (segment (start 136.79 62.79) (end 135.49 64.09) (width 0.2) (layer "F.Cu") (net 13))
 (segment (start 141.986 61.214) (end 140.41 62.79) (width 0.2) (layer "F.Cu") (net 13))
 (segment (start 140.41 62.79) (end 136.79 62.79) (width 0.2) (layer "F.Cu") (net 13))
 (segment (start 146.304 72.438314) (end 146.304 74.5) (width 0.2) (layer "F.Cu") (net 32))
 (segment (start 119.6 68.8) (end 142.665686 68.8) (width 0.2) (layer "F.Cu") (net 32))
 (segment (start 142.665686 68.8) (end 146.304 72.438314) (width 0.2) (layer "F.Cu") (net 32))
 (segment (start 112.88 75.52) (end 119.6 68.8) (width 0.2) (layer "F.Cu") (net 32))
 (segment (start 148.19 73.79) (end 148.9 74.5) (width 0.2) (layer "F.Cu") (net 7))
 (segment (start 148.304 72.104) (end 148.082 71.882) (width 0.2) (layer "F.Cu") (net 7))
 (segment (start 148.304 74.5) (end 148.304 72.104) (width 0.2) (layer "F.Cu") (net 7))
 (segment (start 143.15 66.59) (end 129.35 66.59) (width 0.2) (layer "F.Cu") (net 9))
 (segment (start 145.65 64.09) (end 143.15 66.59) (width 0.2) (layer "F.Cu") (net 9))
 (segment (start 129.35 66.59) (end 123.04 60.28) (width 0.2) (layer "F.Cu") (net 9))
 (segment (start 140.57 71.71) (end 138.46 69.6) (width 0.2) (layer "F.Cu") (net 6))
 (segment (start 138.46 69.6) (end 122.61 69.6) (width 0.2) (layer "F.Cu") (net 6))
 (segment (start 122.61 69.6) (end 116.69 75.52) (width 0.2) (layer "F.Cu") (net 6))
 (segment (start 138.03 64.09) (end 136.73 65.39) (width 0.2) (layer "F.Cu") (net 12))
 (segment (start 136.73 65.39) (end 131.96 65.39) (width 0.2) (layer "F.Cu") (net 12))
 (segment (start 131.96 65.39) (end 126.85 60.28) (width 0.2) (layer "F.Cu") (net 12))
 (segment (start 138.87 65.79) (end 131.09 65.79) (width 0.2) (layer "F.Cu") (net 11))
 (segment (start 131.09 65.79) (end 125.58 60.28) (width 0.2) (layer "F.Cu") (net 11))
 (segment (start 140.57 64.09) (end 138.87 65.79) (width 0.2) (layer "F.Cu") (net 11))
 (segment (start 138.03 71.71) (end 136.33 70.01) (width 0.2) (layer "F.Cu") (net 5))
 (segment (start 136.33 70.01) (end 123.47 70.01) (width 0.2) (layer "F.Cu") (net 5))
 (segment (start 123.47 70.01) (end 117.96 75.52) (width 0.2) (layer "F.Cu") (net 5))
 (segment (start 143.11 64.09) (end 141.01 66.19) (width 0.2) (layer "F.Cu") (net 10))
 (segment (start 130.22 66.19) (end 124.31 60.28) (width 0.2) (layer "F.Cu") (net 10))
 (segment (start 141.01 66.19) (end 130.22 66.19) (width 0.2) (layer "F.Cu") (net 10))
 (segment (start 134.19 70.41) (end 124.34 70.41) (width 0.2) (layer "F.Cu") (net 4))
 (segment (start 124.34 70.41) (end 119.23 75.52) (width 0.2) (layer "F.Cu") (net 4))
 (segment (start 135.49 71.71) (end 134.19 70.41) (width 0.2) (layer "F.Cu") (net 4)))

